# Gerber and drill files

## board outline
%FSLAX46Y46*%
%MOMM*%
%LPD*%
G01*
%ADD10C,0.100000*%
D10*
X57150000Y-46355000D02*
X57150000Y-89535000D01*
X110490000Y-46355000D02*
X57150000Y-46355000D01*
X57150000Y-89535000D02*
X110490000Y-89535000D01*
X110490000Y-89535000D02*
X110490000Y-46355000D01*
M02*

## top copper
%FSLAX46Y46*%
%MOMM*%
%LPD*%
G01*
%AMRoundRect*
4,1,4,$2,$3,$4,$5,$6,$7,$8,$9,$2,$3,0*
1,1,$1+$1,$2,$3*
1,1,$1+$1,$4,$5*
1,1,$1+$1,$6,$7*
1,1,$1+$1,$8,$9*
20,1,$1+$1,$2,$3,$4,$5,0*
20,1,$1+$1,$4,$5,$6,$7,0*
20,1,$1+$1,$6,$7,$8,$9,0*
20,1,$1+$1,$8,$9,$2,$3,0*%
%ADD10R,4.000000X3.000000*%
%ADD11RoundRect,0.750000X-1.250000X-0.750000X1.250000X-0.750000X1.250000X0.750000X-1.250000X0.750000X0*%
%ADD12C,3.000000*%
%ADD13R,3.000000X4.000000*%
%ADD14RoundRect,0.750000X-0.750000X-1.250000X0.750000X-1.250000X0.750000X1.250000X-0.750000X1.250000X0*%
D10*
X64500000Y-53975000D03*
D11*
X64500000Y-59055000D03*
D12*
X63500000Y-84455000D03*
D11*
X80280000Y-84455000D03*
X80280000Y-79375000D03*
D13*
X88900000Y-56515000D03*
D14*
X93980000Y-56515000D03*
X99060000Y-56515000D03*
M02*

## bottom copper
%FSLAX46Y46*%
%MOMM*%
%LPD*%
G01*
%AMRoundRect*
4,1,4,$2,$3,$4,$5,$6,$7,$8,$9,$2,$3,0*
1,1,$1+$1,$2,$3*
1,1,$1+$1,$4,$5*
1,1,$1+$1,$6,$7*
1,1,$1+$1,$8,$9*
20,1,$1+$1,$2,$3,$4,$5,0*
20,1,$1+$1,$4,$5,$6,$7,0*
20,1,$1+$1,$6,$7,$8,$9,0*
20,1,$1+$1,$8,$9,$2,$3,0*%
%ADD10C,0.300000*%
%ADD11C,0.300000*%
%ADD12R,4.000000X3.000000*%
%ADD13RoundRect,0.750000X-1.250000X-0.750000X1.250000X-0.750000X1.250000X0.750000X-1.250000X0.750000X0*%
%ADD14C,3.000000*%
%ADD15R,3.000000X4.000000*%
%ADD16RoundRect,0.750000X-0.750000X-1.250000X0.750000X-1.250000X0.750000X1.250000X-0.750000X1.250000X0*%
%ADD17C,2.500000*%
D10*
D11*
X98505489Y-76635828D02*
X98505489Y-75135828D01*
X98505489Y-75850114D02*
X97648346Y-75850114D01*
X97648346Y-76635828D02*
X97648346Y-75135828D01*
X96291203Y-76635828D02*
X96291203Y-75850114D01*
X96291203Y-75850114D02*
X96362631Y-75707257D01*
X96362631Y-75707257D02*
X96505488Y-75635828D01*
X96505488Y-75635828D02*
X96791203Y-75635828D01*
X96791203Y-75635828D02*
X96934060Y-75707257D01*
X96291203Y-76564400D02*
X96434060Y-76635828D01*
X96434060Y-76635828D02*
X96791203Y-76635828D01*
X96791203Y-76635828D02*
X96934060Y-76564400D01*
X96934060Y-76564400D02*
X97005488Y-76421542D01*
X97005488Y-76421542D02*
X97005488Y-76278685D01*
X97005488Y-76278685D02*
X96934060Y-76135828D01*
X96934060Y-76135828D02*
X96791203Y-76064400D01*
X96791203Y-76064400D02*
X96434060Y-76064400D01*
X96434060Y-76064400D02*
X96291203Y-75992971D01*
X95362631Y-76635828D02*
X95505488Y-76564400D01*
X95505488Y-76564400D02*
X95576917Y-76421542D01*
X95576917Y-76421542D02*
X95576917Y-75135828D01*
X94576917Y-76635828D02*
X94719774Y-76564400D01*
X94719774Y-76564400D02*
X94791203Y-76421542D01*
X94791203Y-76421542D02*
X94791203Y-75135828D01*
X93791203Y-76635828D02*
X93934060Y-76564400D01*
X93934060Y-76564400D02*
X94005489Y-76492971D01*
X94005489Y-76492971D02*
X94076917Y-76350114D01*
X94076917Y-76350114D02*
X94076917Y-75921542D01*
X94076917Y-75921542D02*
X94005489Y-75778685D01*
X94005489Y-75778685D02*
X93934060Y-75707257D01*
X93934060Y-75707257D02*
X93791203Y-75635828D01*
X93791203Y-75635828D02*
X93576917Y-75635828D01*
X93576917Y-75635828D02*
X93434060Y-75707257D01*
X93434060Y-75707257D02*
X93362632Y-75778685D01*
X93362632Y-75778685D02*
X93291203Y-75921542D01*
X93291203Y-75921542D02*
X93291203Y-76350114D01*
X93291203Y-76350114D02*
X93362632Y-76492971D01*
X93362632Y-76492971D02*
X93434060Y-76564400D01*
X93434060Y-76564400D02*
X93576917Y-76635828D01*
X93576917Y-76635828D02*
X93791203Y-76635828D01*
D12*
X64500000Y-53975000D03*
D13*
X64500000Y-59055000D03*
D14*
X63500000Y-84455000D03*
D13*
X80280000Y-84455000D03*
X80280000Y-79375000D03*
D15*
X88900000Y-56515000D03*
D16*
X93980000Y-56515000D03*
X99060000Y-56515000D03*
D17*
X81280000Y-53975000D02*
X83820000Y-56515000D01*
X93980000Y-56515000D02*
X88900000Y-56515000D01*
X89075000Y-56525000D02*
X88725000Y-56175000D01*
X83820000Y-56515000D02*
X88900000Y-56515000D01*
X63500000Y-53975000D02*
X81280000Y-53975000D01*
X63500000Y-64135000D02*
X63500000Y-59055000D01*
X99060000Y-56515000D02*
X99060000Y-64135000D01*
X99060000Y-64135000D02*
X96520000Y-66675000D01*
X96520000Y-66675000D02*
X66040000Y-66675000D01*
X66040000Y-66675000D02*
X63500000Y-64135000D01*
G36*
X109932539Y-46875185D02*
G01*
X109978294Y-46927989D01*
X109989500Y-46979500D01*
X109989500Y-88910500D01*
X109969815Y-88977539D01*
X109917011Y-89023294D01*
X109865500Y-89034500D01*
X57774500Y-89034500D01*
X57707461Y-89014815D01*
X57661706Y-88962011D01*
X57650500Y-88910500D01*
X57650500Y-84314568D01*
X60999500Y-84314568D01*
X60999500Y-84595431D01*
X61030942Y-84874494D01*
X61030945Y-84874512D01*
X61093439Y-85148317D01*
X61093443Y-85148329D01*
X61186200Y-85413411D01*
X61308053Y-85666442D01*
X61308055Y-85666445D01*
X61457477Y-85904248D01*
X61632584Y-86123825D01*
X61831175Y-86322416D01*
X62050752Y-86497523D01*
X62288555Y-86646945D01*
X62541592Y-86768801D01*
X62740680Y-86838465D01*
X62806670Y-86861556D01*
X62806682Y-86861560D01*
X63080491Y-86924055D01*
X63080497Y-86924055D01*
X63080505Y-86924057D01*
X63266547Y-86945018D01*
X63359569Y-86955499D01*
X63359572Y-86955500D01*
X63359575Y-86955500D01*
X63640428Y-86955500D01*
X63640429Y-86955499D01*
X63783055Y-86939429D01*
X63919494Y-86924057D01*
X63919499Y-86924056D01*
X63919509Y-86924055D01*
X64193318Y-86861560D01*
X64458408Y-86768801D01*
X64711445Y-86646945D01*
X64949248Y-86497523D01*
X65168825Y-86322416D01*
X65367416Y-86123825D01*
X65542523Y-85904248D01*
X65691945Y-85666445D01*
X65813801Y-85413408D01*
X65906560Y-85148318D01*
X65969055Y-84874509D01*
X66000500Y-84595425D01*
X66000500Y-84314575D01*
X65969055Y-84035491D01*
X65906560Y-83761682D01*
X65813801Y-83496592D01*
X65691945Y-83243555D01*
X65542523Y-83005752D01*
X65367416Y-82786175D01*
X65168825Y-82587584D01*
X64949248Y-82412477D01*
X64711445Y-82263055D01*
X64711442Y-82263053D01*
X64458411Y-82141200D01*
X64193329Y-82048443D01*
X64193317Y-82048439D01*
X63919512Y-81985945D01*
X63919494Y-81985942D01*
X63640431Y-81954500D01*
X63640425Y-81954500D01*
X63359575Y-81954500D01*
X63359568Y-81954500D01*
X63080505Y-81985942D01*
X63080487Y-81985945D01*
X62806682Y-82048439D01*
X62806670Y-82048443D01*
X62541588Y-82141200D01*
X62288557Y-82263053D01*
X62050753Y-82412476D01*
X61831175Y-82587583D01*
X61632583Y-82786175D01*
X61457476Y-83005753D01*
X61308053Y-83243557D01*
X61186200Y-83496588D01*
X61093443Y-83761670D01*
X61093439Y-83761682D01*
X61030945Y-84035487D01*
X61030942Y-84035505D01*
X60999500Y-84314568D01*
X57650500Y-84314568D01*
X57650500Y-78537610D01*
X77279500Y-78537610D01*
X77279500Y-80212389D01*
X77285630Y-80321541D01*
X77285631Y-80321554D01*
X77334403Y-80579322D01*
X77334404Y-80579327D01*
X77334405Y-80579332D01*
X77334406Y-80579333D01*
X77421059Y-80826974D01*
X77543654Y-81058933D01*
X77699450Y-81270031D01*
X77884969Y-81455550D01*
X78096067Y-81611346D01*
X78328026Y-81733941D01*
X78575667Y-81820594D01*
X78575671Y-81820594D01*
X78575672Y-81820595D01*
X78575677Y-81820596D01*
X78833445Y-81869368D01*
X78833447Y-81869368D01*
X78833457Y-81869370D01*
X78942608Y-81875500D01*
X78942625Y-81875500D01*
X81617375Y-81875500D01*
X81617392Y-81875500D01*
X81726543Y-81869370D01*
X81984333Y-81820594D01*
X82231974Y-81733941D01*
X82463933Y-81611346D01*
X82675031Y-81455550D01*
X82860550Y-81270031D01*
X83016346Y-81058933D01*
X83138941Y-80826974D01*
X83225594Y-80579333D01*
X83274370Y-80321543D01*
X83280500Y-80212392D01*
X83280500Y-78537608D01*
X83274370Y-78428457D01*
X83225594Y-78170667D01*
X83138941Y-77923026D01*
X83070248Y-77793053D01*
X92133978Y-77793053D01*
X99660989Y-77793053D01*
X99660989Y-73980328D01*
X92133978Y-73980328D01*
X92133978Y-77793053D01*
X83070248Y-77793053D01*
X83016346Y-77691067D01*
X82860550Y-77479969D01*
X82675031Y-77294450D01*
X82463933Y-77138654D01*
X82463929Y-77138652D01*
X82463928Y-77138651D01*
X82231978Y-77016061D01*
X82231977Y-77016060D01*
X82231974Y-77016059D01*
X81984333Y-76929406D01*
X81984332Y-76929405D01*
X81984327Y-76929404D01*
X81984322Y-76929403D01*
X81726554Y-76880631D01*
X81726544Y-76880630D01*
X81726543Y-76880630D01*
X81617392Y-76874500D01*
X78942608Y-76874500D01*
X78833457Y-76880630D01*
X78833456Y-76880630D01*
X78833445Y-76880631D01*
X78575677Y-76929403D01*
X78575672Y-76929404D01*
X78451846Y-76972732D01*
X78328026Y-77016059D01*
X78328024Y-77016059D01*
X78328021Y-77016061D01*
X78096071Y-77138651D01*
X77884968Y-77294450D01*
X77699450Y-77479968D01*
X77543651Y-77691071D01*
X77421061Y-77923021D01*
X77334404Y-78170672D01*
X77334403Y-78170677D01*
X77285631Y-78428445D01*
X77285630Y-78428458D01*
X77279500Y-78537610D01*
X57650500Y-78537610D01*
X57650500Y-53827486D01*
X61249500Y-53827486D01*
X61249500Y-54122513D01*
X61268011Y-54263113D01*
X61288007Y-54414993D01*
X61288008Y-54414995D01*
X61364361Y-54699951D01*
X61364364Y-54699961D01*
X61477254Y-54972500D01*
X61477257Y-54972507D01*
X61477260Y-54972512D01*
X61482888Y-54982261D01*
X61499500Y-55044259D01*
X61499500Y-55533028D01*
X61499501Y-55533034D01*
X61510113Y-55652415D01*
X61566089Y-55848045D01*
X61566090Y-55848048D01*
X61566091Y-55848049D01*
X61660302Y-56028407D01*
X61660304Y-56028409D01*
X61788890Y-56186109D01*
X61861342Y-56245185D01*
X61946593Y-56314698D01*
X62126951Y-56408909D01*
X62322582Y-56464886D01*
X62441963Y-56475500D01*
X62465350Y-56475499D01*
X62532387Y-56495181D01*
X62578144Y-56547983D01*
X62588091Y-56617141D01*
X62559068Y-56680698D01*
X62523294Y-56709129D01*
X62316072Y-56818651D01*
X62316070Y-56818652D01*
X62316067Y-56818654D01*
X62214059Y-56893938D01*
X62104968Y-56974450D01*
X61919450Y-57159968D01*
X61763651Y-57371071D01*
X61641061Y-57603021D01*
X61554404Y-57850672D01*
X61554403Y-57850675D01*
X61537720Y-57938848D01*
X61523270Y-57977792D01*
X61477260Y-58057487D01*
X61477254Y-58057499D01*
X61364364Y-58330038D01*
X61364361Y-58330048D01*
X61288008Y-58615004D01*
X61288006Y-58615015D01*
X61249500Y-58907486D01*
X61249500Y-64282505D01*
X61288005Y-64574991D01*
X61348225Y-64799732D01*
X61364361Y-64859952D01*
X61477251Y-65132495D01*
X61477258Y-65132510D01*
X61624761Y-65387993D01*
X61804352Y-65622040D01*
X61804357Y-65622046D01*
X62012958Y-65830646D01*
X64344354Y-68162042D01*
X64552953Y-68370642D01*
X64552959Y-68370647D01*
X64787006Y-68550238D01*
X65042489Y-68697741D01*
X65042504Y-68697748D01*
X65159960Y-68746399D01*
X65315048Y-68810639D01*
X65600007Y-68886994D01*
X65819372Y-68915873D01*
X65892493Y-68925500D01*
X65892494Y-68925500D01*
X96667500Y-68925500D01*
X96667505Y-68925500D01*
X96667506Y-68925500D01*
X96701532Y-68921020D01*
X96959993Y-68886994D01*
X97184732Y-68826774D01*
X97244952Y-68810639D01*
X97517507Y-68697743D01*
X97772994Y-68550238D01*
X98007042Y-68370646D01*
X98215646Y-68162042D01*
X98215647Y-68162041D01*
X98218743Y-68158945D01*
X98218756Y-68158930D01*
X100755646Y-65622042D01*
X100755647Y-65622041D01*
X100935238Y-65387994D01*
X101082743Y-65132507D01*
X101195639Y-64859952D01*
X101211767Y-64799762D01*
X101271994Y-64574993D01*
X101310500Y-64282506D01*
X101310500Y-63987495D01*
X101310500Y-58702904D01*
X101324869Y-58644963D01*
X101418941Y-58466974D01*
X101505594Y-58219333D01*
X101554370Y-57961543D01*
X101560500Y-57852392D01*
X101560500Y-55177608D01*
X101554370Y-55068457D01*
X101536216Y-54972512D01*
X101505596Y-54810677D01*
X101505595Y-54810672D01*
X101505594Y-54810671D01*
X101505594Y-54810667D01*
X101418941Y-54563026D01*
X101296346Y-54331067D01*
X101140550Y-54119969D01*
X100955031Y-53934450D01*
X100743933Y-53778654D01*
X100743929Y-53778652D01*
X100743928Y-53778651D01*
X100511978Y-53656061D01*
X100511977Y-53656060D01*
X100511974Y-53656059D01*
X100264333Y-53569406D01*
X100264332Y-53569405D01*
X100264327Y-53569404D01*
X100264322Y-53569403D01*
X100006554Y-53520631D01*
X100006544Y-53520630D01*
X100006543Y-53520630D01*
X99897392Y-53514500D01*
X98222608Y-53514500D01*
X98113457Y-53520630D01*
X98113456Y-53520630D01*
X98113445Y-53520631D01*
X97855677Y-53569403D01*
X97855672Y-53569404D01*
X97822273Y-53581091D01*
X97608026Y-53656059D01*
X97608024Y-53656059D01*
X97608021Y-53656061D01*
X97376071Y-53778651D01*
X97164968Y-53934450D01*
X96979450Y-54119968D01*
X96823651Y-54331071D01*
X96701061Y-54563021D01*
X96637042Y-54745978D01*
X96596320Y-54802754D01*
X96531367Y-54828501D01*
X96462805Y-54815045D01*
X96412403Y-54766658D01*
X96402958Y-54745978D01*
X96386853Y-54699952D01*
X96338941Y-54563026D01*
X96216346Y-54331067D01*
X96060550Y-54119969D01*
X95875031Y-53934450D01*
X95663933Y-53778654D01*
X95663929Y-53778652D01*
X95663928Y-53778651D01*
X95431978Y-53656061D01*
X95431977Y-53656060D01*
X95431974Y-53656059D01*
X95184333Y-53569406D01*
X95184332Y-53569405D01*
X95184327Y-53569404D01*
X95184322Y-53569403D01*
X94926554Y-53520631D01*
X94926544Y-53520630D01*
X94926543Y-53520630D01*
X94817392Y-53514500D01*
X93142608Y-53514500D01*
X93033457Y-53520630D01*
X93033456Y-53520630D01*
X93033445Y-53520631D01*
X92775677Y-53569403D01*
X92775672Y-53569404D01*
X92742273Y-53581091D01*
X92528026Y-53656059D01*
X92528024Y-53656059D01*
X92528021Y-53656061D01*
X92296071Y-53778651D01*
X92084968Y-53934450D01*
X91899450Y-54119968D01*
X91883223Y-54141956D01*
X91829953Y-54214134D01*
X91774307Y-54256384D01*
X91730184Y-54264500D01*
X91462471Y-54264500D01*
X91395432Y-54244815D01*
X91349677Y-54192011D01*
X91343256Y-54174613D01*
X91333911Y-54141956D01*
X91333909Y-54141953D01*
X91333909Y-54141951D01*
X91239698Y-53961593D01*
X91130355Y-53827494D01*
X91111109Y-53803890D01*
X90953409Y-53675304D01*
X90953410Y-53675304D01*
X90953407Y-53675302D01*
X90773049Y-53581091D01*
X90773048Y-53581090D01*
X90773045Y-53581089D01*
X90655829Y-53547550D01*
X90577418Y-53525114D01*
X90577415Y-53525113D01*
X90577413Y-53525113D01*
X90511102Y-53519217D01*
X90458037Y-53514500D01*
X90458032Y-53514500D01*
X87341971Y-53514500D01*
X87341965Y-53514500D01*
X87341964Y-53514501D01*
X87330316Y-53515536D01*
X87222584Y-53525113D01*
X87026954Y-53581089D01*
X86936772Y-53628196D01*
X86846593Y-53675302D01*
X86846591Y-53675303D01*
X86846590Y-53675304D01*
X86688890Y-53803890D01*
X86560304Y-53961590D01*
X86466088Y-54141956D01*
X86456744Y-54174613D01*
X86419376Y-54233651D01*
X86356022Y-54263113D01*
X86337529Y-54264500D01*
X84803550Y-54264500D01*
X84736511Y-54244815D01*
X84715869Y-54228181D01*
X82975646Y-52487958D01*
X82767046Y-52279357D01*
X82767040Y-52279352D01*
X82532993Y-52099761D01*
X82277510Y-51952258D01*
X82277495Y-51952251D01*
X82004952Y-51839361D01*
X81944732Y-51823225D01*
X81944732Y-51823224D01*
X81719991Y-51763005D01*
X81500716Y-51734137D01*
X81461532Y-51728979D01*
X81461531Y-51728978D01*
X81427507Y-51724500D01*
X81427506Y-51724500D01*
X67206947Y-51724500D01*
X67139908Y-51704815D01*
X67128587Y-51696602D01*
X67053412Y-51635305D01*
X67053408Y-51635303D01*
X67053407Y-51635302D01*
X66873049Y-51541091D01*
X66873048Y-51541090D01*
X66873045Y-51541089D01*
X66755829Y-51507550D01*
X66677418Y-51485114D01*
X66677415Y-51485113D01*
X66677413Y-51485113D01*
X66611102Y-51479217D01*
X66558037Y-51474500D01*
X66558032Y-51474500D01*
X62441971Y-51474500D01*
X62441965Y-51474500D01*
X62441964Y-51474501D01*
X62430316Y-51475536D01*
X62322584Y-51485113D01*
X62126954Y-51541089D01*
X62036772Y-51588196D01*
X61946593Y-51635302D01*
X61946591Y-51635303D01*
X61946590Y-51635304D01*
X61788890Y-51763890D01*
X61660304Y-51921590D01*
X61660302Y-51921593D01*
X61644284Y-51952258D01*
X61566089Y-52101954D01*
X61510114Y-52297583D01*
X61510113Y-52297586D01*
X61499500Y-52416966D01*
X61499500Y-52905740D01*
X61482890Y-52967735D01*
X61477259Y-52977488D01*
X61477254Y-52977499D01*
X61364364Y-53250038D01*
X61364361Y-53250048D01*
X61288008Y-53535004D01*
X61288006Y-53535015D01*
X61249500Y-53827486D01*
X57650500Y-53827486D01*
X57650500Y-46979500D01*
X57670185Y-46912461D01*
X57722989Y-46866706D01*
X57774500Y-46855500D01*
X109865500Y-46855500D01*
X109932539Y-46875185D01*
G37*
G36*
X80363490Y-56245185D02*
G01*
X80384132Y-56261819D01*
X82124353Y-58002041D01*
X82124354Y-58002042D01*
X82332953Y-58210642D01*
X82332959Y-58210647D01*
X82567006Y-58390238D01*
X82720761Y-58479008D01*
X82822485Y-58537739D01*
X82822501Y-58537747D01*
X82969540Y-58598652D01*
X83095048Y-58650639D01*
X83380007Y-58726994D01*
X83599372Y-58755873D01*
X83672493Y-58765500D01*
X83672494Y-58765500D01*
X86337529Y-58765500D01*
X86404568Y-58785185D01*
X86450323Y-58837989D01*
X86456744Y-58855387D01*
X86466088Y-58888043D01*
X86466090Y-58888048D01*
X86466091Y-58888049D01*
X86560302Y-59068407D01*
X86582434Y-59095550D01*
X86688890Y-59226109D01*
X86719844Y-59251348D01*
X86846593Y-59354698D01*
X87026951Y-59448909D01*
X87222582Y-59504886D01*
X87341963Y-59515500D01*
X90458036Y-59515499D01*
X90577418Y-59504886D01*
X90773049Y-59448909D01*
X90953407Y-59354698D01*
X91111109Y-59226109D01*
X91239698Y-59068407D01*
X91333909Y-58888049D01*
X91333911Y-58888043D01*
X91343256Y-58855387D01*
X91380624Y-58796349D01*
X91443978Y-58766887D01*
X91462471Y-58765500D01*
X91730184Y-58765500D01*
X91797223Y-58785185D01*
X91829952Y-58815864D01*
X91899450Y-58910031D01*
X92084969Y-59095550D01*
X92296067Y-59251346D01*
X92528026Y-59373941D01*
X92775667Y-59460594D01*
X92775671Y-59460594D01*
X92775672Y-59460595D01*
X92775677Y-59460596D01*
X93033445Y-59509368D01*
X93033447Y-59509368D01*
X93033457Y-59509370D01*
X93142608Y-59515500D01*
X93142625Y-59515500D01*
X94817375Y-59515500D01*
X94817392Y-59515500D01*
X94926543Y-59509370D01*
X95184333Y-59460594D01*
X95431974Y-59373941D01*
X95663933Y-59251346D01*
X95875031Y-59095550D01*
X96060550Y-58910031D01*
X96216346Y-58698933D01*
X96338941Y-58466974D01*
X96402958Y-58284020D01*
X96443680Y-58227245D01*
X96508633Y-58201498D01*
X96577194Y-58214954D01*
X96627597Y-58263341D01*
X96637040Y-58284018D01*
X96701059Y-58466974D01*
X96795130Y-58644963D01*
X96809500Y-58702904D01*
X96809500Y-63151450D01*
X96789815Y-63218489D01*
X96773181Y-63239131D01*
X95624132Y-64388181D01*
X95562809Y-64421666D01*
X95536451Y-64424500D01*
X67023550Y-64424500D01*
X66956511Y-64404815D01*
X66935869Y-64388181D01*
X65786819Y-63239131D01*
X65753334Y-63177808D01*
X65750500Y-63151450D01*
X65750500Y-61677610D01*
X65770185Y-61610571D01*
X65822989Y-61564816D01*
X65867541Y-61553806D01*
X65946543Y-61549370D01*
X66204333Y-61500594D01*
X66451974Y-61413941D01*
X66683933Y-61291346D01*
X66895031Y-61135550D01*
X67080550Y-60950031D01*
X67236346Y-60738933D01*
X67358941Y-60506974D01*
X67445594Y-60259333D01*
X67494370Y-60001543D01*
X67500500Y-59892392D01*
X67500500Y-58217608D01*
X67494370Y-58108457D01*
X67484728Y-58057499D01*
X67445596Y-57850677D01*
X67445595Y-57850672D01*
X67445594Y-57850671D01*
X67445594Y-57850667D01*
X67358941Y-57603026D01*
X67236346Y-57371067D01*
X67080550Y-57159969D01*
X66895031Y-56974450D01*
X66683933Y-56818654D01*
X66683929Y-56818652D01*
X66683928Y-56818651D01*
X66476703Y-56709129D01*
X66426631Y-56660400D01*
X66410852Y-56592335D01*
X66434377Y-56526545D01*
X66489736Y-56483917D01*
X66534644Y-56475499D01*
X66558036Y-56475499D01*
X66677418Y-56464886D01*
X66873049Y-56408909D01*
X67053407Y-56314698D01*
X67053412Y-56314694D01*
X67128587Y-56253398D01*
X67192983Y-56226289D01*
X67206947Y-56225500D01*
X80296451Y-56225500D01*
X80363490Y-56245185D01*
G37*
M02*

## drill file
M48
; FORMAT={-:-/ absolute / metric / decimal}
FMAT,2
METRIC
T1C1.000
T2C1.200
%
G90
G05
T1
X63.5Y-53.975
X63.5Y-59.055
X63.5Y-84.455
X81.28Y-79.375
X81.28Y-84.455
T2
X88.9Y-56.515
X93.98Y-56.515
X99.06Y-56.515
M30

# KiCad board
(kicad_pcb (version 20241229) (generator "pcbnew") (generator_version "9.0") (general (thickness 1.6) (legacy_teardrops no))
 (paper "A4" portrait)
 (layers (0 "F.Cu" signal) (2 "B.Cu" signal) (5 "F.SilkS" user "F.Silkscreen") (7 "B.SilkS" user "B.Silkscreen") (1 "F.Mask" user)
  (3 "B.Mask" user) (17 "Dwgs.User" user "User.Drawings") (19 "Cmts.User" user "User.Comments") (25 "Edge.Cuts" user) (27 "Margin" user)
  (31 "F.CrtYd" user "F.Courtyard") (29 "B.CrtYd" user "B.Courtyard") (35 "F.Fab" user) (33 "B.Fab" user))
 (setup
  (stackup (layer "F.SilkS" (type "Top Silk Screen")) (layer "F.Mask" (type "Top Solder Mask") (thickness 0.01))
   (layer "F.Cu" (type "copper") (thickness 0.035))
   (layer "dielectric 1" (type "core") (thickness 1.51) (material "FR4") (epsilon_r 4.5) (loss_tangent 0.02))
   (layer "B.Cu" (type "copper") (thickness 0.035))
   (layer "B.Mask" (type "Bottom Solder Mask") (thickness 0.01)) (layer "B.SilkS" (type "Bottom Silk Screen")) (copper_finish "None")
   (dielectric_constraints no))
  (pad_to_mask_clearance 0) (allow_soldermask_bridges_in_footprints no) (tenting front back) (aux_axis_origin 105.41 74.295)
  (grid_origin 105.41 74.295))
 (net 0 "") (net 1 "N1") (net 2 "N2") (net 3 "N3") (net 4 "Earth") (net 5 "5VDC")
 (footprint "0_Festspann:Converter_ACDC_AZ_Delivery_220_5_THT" (layer "F.Cu") (at 63.5 53.975)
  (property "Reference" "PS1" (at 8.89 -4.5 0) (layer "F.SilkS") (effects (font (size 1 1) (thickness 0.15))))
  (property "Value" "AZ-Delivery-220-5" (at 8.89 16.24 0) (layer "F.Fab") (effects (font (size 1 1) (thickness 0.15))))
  (pad "1" thru_hole rect (at 0 0) (size 4 3) (drill 1 (offset 1 0)) (layers "*.Cu" "*.Mask") (remove_unused_layers no) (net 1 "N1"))
  (pad "3" thru_hole roundrect (at 0 5.08) (size 4 3) (drill 1 (offset 1 0)) (layers "*.Cu" "*.Mask") (remove_unused_layers no)
   (roundrect_rratio 0.25) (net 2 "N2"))
  (pad "5" thru_hole circle (at 0 30.48) (size 3 3) (drill 1) (layers "*.Cu" "*.Mask") (remove_unused_layers no) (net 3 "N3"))
  (pad "14" thru_hole roundrect (at 17.78 30.48) (size 4 3) (drill 1 (offset -1 0)) (layers "*.Cu" "*.Mask") (remove_unused_layers no)
   (roundrect_rratio 0.25) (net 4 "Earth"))
  (pad "16" thru_hole roundrect (at 17.78 25.4) (size 4 3) (drill 1 (offset -1 0)) (layers "*.Cu" "*.Mask") (remove_unused_layers no)
   (roundrect_rratio 0.25) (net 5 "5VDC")))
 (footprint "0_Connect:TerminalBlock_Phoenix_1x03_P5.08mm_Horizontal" (layer "F.Cu") (at 88.9 56.515)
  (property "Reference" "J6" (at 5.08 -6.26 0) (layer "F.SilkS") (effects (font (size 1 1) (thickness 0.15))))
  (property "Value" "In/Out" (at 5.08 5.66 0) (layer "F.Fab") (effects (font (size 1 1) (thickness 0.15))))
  (pad "1" thru_hole rect (at 0 0) (size 3 4) (drill 1.2) (layers "*.Cu" "*.Mask") (remove_unused_layers no) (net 1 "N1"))
  (pad "2" thru_hole roundrect (at 5.08 0) (size 3 4) (drill 1.2) (layers "*.Cu" "*.Mask") (remove_unused_layers no) (roundrect_rratio 0.25)
   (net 1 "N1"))
  (pad "3" thru_hole roundrect (at 10.16 0) (size 3 4) (drill 1.2) (layers "*.Cu" "*.Mask") (remove_unused_layers no)
   (roundrect_rratio 0.25) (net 2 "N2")))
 (gr_line (start 57.15 46.355) (end 57.15 89.535) (stroke (width 0.1) (type default)) (layer "Edge.Cuts"))
 (gr_line (start 110.49 46.355) (end 57.15 46.355) (stroke (width 0.1) (type default)) (layer "Edge.Cuts"))
 (gr_line (start 57.15 89.535) (end 110.49 89.535) (stroke (width 0.1) (type default)) (layer "Edge.Cuts"))
 (gr_line (start 110.49 89.535) (end 110.49 46.355) (stroke (width 0.1) (type default)) (layer "Edge.Cuts"))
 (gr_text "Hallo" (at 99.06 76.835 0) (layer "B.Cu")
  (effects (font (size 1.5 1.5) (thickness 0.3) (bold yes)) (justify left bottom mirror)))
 (segment (start 81.28 53.975) (end 83.82 56.515) (width 2.5) (layer "B.Cu") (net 1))
 (segment (start 93.98 56.515) (end 88.9 56.515) (width 2.5) (layer "B.Cu") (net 1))
 (segment (start 89.075 56.525) (end 88.725 56.175) (width 2.5) (layer "B.Cu") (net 1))
 (segment (start 83.82 56.515) (end 88.9 56.515) (width 2.5) (layer "B.Cu") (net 1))
 (segment (start 63.5 53.975) (end 81.28 53.975) (width 2.5) (layer "B.Cu") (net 1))
 (segment (start 63.5 64.135) (end 63.5 59.055) (width 2.5) (layer "B.Cu") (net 2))
 (segment (start 99.06 56.515) (end 99.06 64.135) (width 2.5) (layer "B.Cu") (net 2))
 (segment (start 99.06 64.135) (end 96.52 66.675) (width 2.5) (layer "B.Cu") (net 2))
 (segment (start 96.52 66.675) (end 66.04 66.675) (width 2.5) (layer "B.Cu") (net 2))
 (segment (start 66.04 66.675) (end 63.5 64.135) (width 2.5) (layer "B.Cu") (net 2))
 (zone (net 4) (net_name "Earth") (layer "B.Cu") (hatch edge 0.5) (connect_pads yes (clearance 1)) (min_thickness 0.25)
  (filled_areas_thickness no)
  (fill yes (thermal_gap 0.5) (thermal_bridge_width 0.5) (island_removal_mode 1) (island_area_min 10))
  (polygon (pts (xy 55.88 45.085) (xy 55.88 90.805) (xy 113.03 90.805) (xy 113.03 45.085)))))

